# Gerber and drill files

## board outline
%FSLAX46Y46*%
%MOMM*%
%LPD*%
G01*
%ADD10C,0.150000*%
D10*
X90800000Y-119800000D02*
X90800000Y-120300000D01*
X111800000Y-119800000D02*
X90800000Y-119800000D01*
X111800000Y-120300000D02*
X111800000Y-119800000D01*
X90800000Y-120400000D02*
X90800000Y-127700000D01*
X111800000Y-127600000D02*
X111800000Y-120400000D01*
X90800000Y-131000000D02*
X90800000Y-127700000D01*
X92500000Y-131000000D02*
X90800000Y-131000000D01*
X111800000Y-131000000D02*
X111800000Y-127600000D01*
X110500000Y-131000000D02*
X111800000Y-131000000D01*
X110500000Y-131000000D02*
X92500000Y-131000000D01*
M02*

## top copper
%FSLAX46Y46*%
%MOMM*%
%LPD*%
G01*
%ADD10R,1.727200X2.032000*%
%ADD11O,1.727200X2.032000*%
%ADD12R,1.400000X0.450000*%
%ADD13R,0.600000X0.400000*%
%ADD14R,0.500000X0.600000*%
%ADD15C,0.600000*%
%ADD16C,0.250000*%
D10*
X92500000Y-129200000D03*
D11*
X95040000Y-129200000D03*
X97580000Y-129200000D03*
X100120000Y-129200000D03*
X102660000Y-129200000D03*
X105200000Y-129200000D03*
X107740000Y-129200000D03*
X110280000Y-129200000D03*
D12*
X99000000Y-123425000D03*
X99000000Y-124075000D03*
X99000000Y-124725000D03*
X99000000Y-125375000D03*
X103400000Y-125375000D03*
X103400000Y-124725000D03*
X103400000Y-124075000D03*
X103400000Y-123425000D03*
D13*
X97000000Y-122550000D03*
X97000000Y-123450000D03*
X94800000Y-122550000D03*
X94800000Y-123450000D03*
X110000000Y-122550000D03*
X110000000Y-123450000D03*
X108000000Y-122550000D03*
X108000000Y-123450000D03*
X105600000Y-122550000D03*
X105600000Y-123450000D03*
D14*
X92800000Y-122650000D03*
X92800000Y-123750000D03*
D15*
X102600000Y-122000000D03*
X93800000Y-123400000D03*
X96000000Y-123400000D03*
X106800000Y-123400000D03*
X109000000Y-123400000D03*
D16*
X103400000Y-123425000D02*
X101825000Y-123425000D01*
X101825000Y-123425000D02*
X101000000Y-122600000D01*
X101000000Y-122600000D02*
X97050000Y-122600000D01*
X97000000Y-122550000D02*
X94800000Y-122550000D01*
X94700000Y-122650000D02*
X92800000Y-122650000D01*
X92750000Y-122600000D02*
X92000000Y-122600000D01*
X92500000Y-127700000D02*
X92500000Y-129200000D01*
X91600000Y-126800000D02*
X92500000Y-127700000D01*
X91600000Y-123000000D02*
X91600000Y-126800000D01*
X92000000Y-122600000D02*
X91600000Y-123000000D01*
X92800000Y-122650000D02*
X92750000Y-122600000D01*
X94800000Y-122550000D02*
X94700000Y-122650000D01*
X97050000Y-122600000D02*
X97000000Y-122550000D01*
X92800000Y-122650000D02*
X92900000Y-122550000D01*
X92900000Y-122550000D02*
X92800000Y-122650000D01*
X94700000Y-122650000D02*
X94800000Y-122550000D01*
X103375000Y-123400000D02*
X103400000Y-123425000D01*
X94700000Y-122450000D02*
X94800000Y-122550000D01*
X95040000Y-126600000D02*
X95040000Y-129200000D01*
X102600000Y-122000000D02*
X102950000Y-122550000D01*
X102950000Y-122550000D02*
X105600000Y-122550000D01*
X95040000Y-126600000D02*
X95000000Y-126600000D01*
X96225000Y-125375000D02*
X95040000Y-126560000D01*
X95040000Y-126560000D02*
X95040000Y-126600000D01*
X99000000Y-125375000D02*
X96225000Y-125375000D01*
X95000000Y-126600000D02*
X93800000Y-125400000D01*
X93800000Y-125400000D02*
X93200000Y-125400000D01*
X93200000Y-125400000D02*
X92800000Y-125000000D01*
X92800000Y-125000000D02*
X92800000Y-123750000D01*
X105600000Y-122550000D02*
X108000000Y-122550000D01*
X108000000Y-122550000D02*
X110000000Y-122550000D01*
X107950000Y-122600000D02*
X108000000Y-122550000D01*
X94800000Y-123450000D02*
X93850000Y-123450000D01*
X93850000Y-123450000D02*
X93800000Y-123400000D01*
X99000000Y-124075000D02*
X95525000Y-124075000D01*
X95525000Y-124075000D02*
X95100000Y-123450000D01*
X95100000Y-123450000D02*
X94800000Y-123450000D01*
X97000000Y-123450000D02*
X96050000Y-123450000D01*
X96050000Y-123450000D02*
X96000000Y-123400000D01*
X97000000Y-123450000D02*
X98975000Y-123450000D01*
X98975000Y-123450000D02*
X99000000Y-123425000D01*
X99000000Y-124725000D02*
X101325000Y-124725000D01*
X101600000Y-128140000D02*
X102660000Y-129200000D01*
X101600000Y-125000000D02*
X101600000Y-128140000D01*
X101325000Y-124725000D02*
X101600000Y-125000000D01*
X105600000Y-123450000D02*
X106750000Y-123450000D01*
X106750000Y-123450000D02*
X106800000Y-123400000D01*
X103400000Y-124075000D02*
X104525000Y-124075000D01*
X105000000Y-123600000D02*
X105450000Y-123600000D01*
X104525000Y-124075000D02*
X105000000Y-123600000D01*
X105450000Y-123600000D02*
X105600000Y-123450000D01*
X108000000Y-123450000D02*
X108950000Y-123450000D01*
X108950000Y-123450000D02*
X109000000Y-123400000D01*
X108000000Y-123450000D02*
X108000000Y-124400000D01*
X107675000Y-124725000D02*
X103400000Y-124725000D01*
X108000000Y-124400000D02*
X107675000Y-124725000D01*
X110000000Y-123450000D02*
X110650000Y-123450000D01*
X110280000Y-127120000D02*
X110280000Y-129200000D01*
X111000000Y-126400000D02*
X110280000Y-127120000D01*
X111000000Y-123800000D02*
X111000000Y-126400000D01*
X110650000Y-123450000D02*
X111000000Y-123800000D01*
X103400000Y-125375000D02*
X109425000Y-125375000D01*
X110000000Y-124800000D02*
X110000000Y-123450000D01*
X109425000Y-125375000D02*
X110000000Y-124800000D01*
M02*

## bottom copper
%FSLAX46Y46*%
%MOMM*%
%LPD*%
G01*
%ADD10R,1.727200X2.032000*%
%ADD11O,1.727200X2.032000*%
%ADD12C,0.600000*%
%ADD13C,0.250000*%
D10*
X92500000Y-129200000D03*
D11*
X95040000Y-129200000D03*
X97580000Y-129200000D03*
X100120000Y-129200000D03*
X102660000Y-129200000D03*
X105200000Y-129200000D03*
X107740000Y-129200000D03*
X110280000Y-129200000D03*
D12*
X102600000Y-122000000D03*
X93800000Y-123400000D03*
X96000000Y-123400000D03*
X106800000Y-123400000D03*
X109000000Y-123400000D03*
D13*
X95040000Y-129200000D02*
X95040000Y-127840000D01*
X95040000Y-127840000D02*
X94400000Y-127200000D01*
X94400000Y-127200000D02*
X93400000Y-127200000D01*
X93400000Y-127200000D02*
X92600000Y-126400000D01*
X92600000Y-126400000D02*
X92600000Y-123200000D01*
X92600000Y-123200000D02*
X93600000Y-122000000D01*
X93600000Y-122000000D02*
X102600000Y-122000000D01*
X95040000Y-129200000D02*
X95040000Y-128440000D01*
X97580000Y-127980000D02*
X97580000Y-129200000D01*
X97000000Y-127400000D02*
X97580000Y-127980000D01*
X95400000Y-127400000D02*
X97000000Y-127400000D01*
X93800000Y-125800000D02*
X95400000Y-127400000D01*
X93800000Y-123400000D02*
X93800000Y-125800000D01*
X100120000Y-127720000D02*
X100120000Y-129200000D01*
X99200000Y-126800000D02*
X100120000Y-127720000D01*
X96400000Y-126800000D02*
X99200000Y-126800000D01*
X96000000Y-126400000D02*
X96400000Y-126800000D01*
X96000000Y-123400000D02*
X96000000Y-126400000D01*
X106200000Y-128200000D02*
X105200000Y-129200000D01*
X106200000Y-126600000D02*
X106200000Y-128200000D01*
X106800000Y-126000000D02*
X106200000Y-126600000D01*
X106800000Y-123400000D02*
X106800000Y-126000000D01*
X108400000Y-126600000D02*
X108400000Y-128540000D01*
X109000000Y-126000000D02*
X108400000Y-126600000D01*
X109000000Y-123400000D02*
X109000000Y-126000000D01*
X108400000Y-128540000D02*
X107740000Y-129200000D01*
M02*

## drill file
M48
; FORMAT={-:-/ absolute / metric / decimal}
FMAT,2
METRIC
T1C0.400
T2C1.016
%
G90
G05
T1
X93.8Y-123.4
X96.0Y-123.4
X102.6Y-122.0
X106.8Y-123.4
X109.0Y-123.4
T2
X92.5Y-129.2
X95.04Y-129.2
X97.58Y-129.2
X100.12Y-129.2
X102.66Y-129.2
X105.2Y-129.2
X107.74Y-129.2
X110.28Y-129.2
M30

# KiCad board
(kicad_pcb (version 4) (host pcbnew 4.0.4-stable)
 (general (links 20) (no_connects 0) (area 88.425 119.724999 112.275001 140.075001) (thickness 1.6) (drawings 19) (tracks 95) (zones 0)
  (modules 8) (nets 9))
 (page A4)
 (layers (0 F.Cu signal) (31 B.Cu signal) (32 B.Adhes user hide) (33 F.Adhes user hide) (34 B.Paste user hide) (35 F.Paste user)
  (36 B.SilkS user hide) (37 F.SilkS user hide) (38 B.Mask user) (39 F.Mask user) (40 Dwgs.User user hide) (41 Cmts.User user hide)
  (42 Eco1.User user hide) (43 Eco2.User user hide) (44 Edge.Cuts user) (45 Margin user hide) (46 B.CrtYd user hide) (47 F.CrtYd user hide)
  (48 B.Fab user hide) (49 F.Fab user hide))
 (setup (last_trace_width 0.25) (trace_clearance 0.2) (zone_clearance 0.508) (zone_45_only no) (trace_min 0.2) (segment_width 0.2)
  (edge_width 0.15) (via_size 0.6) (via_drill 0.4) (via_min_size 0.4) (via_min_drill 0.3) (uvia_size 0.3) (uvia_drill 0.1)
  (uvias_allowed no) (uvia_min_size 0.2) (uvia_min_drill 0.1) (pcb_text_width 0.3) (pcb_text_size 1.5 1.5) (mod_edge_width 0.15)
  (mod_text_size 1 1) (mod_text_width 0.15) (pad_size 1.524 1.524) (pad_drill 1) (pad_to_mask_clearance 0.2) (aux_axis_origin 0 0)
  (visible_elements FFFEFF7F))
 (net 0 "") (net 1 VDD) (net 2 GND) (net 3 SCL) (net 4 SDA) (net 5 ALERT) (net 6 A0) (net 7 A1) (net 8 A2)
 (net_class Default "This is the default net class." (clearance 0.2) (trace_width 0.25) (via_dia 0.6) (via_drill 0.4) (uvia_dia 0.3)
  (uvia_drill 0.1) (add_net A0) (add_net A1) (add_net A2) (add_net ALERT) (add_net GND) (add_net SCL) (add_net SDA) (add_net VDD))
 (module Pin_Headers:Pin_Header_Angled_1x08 (layer B.Cu) (at 92.5 129.2 270)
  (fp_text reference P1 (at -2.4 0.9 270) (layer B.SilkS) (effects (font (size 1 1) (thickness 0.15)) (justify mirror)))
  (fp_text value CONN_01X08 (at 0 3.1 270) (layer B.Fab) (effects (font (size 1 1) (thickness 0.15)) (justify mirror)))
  (pad 1 thru_hole rect (at 0 0 270) (size 2.032 1.7272) (drill 1.016) (layers *.Cu *.Mask) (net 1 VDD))
  (pad 2 thru_hole oval (at 0 -2.54 270) (size 2.032 1.7272) (drill 1.016) (layers *.Cu *.Mask) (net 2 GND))
  (pad 3 thru_hole oval (at 0 -5.08 270) (size 2.032 1.7272) (drill 1.016) (layers *.Cu *.Mask) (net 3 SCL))
  (pad 4 thru_hole oval (at 0 -7.62 270) (size 2.032 1.7272) (drill 1.016) (layers *.Cu *.Mask) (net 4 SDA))
  (pad 5 thru_hole oval (at 0 -10.16 270) (size 2.032 1.7272) (drill 1.016) (layers *.Cu *.Mask) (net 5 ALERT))
  (pad 6 thru_hole oval (at 0 -12.7 270) (size 2.032 1.7272) (drill 1.016) (layers *.Cu *.Mask) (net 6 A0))
  (pad 7 thru_hole oval (at 0 -15.24 270) (size 2.032 1.7272) (drill 1.016) (layers *.Cu *.Mask) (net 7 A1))
  (pad 8 thru_hole oval (at 0 -17.78 270) (size 2.032 1.7272) (drill 1.016) (layers *.Cu *.Mask) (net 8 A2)))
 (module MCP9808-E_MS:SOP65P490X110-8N (layer F.Cu) (at 101.2 124.4) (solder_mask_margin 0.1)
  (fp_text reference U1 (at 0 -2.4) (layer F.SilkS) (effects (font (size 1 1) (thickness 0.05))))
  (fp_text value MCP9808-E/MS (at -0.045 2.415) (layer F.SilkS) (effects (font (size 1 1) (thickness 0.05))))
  (pad 1 smd rect (at -2.2 -0.975) (size 1.4 0.45) (layers F.Cu F.Paste F.Mask) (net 4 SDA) (solder_mask_margin 0.2))
  (pad 2 smd rect (at -2.2 -0.325) (size 1.4 0.45) (layers F.Cu F.Paste F.Mask) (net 3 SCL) (solder_mask_margin 0.2))
  (pad 3 smd rect (at -2.2 0.325) (size 1.4 0.45) (layers F.Cu F.Paste F.Mask) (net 5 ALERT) (solder_mask_margin 0.2))
  (pad 4 smd rect (at -2.2 0.975) (size 1.4 0.45) (layers F.Cu F.Paste F.Mask) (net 2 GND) (solder_mask_margin 0.2))
  (pad 5 smd rect (at 2.2 0.975 180) (size 1.4 0.45) (layers F.Cu F.Paste F.Mask) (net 8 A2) (solder_mask_margin 0.2))
  (pad 6 smd rect (at 2.2 0.325 180) (size 1.4 0.45) (layers F.Cu F.Paste F.Mask) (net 7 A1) (solder_mask_margin 0.2))
  (pad 7 smd rect (at 2.2 -0.325 180) (size 1.4 0.45) (layers F.Cu F.Paste F.Mask) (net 6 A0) (solder_mask_margin 0.2))
  (pad 8 smd rect (at 2.2 -0.975 180) (size 1.4 0.45) (layers F.Cu F.Paste F.Mask) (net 1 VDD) (solder_mask_margin 0.2)))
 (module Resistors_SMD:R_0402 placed (layer F.Cu) (at 97 123 270)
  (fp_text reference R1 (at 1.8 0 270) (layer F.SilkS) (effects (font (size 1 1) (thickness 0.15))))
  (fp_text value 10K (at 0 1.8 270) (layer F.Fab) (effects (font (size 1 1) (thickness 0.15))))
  (pad 1 smd rect (at -0.45 0 270) (size 0.4 0.6) (layers F.Cu F.Paste F.Mask) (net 1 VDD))
  (pad 2 smd rect (at 0.45 0 270) (size 0.4 0.6) (layers F.Cu F.Paste F.Mask) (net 4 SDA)))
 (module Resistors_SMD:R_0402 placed (layer F.Cu) (at 94.8 123 270)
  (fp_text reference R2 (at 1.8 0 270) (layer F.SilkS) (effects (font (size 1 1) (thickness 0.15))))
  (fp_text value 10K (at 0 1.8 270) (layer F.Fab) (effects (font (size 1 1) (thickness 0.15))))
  (pad 1 smd rect (at -0.45 0 270) (size 0.4 0.6) (layers F.Cu F.Paste F.Mask) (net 1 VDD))
  (pad 2 smd rect (at 0.45 0 270) (size 0.4 0.6) (layers F.Cu F.Paste F.Mask) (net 3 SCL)))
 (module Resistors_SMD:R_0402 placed (layer F.Cu) (at 110 123 270)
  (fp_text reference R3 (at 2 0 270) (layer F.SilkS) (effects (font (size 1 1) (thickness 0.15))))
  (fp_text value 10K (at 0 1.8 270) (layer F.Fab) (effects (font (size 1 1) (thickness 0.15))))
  (pad 1 smd rect (at -0.45 0 270) (size 0.4 0.6) (layers F.Cu F.Paste F.Mask) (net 2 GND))
  (pad 2 smd rect (at 0.45 0 270) (size 0.4 0.6) (layers F.Cu F.Paste F.Mask) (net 8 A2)))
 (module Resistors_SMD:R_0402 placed (layer F.Cu) (at 108 123 270)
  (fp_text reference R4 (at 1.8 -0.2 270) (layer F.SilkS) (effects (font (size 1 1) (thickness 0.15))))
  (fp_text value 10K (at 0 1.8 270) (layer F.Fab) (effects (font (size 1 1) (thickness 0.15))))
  (pad 1 smd rect (at -0.45 0 270) (size 0.4 0.6) (layers F.Cu F.Paste F.Mask) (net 2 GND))
  (pad 2 smd rect (at 0.45 0 270) (size 0.4 0.6) (layers F.Cu F.Paste F.Mask) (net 7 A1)))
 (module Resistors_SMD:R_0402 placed (layer F.Cu) (at 105.6 123 270)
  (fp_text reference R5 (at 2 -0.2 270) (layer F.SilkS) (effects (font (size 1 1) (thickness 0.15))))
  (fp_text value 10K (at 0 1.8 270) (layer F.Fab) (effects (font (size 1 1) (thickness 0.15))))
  (pad 1 smd rect (at -0.45 0 270) (size 0.4 0.6) (layers F.Cu F.Paste F.Mask) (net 2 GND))
  (pad 2 smd rect (at 0.45 0 270) (size 0.4 0.6) (layers F.Cu F.Paste F.Mask) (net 6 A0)))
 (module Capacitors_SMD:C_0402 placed (layer F.Cu) (at 92.8 123.2 270)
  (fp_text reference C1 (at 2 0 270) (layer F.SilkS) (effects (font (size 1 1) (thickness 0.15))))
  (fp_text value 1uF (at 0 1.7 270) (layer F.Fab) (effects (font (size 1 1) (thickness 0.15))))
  (pad 1 smd rect (at -0.55 0 270) (size 0.6 0.5) (layers F.Cu F.Paste F.Mask) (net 1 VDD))
  (pad 2 smd rect (at 0.55 0 270) (size 0.6 0.5) (layers F.Cu F.Paste F.Mask) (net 2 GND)))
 (gr_line (start 90.8 119.8) (end 90.8 120.3) (angle 90) (layer Edge.Cuts) (width 0.15))
 (gr_line (start 111.8 119.8) (end 90.8 119.8) (angle 90) (layer Edge.Cuts) (width 0.15))
 (gr_line (start 111.8 120.3) (end 111.8 119.8) (angle 90) (layer Edge.Cuts) (width 0.15))
 (gr_line (start 90.8 120.4) (end 90.8 127.7) (angle 90) (layer Edge.Cuts) (width 0.15))
 (gr_line (start 111.8 127.6) (end 111.8 120.4) (angle 90) (layer Edge.Cuts) (width 0.15))
 (gr_line (start 90.8 131) (end 90.8 127.7) (angle 90) (layer Edge.Cuts) (width 0.15))
 (gr_line (start 92.5 131) (end 90.8 131) (angle 90) (layer Edge.Cuts) (width 0.15))
 (gr_line (start 111.8 131) (end 111.8 127.6) (angle 90) (layer Edge.Cuts) (width 0.15))
 (gr_line (start 110.5 131) (end 111.8 131) (angle 90) (layer Edge.Cuts) (width 0.15))
 (gr_line (start 110.5 131) (end 92.5 131) (angle 90) (layer Edge.Cuts) (width 0.15))
 (segment (start 103.4 123.425) (end 101.825 123.425) (width 0.25) (layer F.Cu) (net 1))
 (segment (start 101.825 123.425) (end 101 122.6) (width 0.25) (layer F.Cu) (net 1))
 (segment (start 101 122.6) (end 97.05 122.6) (width 0.25) (layer F.Cu) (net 1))
 (segment (start 97 122.55) (end 94.8 122.55) (width 0.25) (layer F.Cu) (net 1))
 (segment (start 94.7 122.65) (end 92.8 122.65) (width 0.25) (layer F.Cu) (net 1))
 (segment (start 92.75 122.6) (end 92 122.6) (width 0.25) (layer F.Cu) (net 1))
 (segment (start 92.5 127.7) (end 92.5 129.2) (width 0.25) (layer F.Cu) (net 1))
 (segment (start 91.6 126.8) (end 92.5 127.7) (width 0.25) (layer F.Cu) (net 1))
 (segment (start 91.6 123) (end 91.6 126.8) (width 0.25) (layer F.Cu) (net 1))
 (segment (start 92 122.6) (end 91.6 123) (width 0.25) (layer F.Cu) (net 1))
 (segment (start 92.8 122.65) (end 92.75 122.6) (width 0.25) (layer F.Cu) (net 1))
 (segment (start 94.8 122.55) (end 94.7 122.65) (width 0.25) (layer F.Cu) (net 1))
 (segment (start 97.05 122.6) (end 97 122.55) (width 0.25) (layer F.Cu) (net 1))
 (segment (start 92.8 122.65) (end 92.9 122.55) (width 0.25) (layer F.Cu) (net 1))
 (segment (start 92.9 122.55) (end 92.8 122.65) (width 0.25) (layer F.Cu) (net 1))
 (segment (start 94.7 122.65) (end 94.8 122.55) (width 0.25) (layer F.Cu) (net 1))
 (segment (start 103.375 123.4) (end 103.4 123.425) (width 0.25) (layer F.Cu) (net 1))
 (segment (start 94.7 122.45) (end 94.8 122.55) (width 0.25) (layer F.Cu) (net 1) (status 30))
 (segment (start 95.04 126.6) (end 95.04 129.2) (width 0.25) (layer F.Cu) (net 2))
 (segment (start 95.04 129.2) (end 95.04 127.84) (width 0.25) (layer B.Cu) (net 2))
 (segment (start 95.04 127.84) (end 94.4 127.2) (width 0.25) (layer B.Cu) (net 2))
 (segment (start 94.4 127.2) (end 93.4 127.2) (width 0.25) (layer B.Cu) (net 2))
 (segment (start 93.4 127.2) (end 92.6 126.4) (width 0.25) (layer B.Cu) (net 2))
 (segment (start 92.6 126.4) (end 92.6 123.2) (width 0.25) (layer B.Cu) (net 2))
 (segment (start 92.6 123.2) (end 93.6 122) (width 0.25) (layer B.Cu) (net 2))
 (segment (start 93.6 122) (end 102.6 122) (width 0.25) (layer B.Cu) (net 2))
 (via (at 102.6 122) (size 0.6) (drill 0.4) (layers F.Cu B.Cu) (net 2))
 (segment (start 102.6 122) (end 102.95 122.55) (width 0.25) (layer F.Cu) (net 2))
 (segment (start 102.95 122.55) (end 105.6 122.55) (width 0.25) (layer F.Cu) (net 2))
 (segment (start 95.04 129.2) (end 95.04 128.44) (width 0.25) (layer B.Cu) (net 2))
 (segment (start 95.04 126.6) (end 95 126.6) (width 0.25) (layer F.Cu) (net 2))
 (segment (start 96.225 125.375) (end 95.04 126.56) (width 0.25) (layer F.Cu) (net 2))
 (segment (start 95.04 126.56) (end 95.04 126.6) (width 0.25) (layer F.Cu) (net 2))
 (segment (start 99 125.375) (end 96.225 125.375) (width 0.25) (layer F.Cu) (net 2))
 (segment (start 95 126.6) (end 93.8 125.4) (width 0.25) (layer F.Cu) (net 2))
 (segment (start 93.8 125.4) (end 93.2 125.4) (width 0.25) (layer F.Cu) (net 2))
 (segment (start 93.2 125.4) (end 92.8 125) (width 0.25) (layer F.Cu) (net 2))
 (segment (start 92.8 125) (end 92.8 123.75) (width 0.25) (layer F.Cu) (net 2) (status 20))
 (segment (start 105.6 122.55) (end 108 122.55) (width 0.25) (layer F.Cu) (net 2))
 (segment (start 108 122.55) (end 110 122.55) (width 0.25) (layer F.Cu) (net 2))
 (segment (start 107.95 122.6) (end 108 122.55) (width 0.25) (layer F.Cu) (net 2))
 (segment (start 94.8 123.45) (end 93.85 123.45) (width 0.25) (layer F.Cu) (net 3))
 (segment (start 97.58 127.98) (end 97.58 129.2) (width 0.25) (layer B.Cu) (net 3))
 (segment (start 97 127.4) (end 97.58 127.98) (width 0.25) (layer B.Cu) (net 3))
 (segment (start 95.4 127.4) (end 97 127.4) (width 0.25) (layer B.Cu) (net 3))
 (segment (start 93.8 125.8) (end 95.4 127.4) (width 0.25) (layer B.Cu) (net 3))
 (segment (start 93.8 123.4) (end 93.8 125.8) (width 0.25) (layer B.Cu) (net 3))
 (via (at 93.8 123.4) (size 0.6) (drill 0.4) (layers F.Cu B.Cu) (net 3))
 (segment (start 93.85 123.45) (end 93.8 123.4) (width 0.25) (layer F.Cu) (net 3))
 (segment (start 99 124.075) (end 95.525 124.075) (width 0.25) (layer F.Cu) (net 3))
 (segment (start 95.525 124.075) (end 95.1 123.45) (width 0.25) (layer F.Cu) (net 3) (status 20))
 (segment (start 95.1 123.45) (end 94.8 123.45) (width 0.25) (layer F.Cu) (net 3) (status 30))
 (segment (start 97 123.45) (end 96.05 123.45) (width 0.25) (layer F.Cu) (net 4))
 (segment (start 100.12 127.72) (end 100.12 129.2) (width 0.25) (layer B.Cu) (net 4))
 (segment (start 99.2 126.8) (end 100.12 127.72) (width 0.25) (layer B.Cu) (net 4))
 (segment (start 96.4 126.8) (end 99.2 126.8) (width 0.25) (layer B.Cu) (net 4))
 (segment (start 96 126.4) (end 96.4 126.8) (width 0.25) (layer B.Cu) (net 4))
 (segment (start 96 123.4) (end 96 126.4) (width 0.25) (layer B.Cu) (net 4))
 (via (at 96 123.4) (size 0.6) (drill 0.4) (layers F.Cu B.Cu) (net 4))
 (segment (start 96.05 123.45) (end 96 123.4) (width 0.25) (layer F.Cu) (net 4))
 (segment (start 97 123.45) (end 98.975 123.45) (width 0.25) (layer F.Cu) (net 4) (status 10))
 (segment (start 98.975 123.45) (end 99 123.425) (width 0.25) (layer F.Cu) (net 4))
 (segment (start 99 124.725) (end 101.325 124.725) (width 0.25) (layer F.Cu) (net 5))
 (segment (start 101.6 128.14) (end 102.66 129.2) (width 0.25) (layer F.Cu) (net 5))
 (segment (start 101.6 125) (end 101.6 128.14) (width 0.25) (layer F.Cu) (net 5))
 (segment (start 101.325 124.725) (end 101.6 125) (width 0.25) (layer F.Cu) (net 5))
 (segment (start 105.6 123.45) (end 106.75 123.45) (width 0.25) (layer F.Cu) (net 6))
 (segment (start 106.2 128.2) (end 105.2 129.2) (width 0.25) (layer B.Cu) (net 6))
 (segment (start 106.2 126.6) (end 106.2 128.2) (width 0.25) (layer B.Cu) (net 6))
 (segment (start 106.8 126) (end 106.2 126.6) (width 0.25) (layer B.Cu) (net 6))
 (segment (start 106.8 123.4) (end 106.8 126) (width 0.25) (layer B.Cu) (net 6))
 (via (at 106.8 123.4) (size 0.6) (drill 0.4) (layers F.Cu B.Cu) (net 6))
 (segment (start 106.75 123.45) (end 106.8 123.4) (width 0.25) (layer F.Cu) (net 6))
 (segment (start 103.4 124.075) (end 104.525 124.075) (width 0.25) (layer F.Cu) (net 6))
 (segment (start 105 123.6) (end 105.45 123.6) (width 0.25) (layer F.Cu) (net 6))
 (segment (start 104.525 124.075) (end 105 123.6) (width 0.25) (layer F.Cu) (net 6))
 (segment (start 105.45 123.6) (end 105.6 123.45) (width 0.25) (layer F.Cu) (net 6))
 (segment (start 108 123.45) (end 108.95 123.45) (width 0.25) (layer F.Cu) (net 7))
 (segment (start 108.4 126.6) (end 108.4 128.54) (width 0.25) (layer B.Cu) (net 7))
 (segment (start 109 126) (end 108.4 126.6) (width 0.25) (layer B.Cu) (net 7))
 (segment (start 109 123.4) (end 109 126) (width 0.25) (layer B.Cu) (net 7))
 (via (at 109 123.4) (size 0.6) (drill 0.4) (layers F.Cu B.Cu) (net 7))
 (segment (start 108.95 123.45) (end 109 123.4) (width 0.25) (layer F.Cu) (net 7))
 (segment (start 108.4 128.54) (end 107.74 129.2) (width 0.25) (layer B.Cu) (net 7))
 (segment (start 108 123.45) (end 108 124.4) (width 0.25) (layer F.Cu) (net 7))
 (segment (start 107.675 124.725) (end 103.4 124.725) (width 0.25) (layer F.Cu) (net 7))
 (segment (start 108 124.4) (end 107.675 124.725) (width 0.25) (layer F.Cu) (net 7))
 (segment (start 110 123.45) (end 110.65 123.45) (width 0.25) (layer F.Cu) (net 8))
 (segment (start 110.28 127.12) (end 110.28 129.2) (width 0.25) (layer F.Cu) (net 8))
 (segment (start 111 126.4) (end 110.28 127.12) (width 0.25) (layer F.Cu) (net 8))
 (segment (start 111 123.8) (end 111 126.4) (width 0.25) (layer F.Cu) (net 8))
 (segment (start 110.65 123.45) (end 111 123.8) (width 0.25) (layer F.Cu) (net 8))
 (segment (start 103.4 125.375) (end 109.425 125.375) (width 0.25) (layer F.Cu) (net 8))
 (segment (start 110 124.8) (end 110 123.45) (width 0.25) (layer F.Cu) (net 8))
 (segment (start 109.425 125.375) (end 110 124.8) (width 0.25) (layer F.Cu) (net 8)))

